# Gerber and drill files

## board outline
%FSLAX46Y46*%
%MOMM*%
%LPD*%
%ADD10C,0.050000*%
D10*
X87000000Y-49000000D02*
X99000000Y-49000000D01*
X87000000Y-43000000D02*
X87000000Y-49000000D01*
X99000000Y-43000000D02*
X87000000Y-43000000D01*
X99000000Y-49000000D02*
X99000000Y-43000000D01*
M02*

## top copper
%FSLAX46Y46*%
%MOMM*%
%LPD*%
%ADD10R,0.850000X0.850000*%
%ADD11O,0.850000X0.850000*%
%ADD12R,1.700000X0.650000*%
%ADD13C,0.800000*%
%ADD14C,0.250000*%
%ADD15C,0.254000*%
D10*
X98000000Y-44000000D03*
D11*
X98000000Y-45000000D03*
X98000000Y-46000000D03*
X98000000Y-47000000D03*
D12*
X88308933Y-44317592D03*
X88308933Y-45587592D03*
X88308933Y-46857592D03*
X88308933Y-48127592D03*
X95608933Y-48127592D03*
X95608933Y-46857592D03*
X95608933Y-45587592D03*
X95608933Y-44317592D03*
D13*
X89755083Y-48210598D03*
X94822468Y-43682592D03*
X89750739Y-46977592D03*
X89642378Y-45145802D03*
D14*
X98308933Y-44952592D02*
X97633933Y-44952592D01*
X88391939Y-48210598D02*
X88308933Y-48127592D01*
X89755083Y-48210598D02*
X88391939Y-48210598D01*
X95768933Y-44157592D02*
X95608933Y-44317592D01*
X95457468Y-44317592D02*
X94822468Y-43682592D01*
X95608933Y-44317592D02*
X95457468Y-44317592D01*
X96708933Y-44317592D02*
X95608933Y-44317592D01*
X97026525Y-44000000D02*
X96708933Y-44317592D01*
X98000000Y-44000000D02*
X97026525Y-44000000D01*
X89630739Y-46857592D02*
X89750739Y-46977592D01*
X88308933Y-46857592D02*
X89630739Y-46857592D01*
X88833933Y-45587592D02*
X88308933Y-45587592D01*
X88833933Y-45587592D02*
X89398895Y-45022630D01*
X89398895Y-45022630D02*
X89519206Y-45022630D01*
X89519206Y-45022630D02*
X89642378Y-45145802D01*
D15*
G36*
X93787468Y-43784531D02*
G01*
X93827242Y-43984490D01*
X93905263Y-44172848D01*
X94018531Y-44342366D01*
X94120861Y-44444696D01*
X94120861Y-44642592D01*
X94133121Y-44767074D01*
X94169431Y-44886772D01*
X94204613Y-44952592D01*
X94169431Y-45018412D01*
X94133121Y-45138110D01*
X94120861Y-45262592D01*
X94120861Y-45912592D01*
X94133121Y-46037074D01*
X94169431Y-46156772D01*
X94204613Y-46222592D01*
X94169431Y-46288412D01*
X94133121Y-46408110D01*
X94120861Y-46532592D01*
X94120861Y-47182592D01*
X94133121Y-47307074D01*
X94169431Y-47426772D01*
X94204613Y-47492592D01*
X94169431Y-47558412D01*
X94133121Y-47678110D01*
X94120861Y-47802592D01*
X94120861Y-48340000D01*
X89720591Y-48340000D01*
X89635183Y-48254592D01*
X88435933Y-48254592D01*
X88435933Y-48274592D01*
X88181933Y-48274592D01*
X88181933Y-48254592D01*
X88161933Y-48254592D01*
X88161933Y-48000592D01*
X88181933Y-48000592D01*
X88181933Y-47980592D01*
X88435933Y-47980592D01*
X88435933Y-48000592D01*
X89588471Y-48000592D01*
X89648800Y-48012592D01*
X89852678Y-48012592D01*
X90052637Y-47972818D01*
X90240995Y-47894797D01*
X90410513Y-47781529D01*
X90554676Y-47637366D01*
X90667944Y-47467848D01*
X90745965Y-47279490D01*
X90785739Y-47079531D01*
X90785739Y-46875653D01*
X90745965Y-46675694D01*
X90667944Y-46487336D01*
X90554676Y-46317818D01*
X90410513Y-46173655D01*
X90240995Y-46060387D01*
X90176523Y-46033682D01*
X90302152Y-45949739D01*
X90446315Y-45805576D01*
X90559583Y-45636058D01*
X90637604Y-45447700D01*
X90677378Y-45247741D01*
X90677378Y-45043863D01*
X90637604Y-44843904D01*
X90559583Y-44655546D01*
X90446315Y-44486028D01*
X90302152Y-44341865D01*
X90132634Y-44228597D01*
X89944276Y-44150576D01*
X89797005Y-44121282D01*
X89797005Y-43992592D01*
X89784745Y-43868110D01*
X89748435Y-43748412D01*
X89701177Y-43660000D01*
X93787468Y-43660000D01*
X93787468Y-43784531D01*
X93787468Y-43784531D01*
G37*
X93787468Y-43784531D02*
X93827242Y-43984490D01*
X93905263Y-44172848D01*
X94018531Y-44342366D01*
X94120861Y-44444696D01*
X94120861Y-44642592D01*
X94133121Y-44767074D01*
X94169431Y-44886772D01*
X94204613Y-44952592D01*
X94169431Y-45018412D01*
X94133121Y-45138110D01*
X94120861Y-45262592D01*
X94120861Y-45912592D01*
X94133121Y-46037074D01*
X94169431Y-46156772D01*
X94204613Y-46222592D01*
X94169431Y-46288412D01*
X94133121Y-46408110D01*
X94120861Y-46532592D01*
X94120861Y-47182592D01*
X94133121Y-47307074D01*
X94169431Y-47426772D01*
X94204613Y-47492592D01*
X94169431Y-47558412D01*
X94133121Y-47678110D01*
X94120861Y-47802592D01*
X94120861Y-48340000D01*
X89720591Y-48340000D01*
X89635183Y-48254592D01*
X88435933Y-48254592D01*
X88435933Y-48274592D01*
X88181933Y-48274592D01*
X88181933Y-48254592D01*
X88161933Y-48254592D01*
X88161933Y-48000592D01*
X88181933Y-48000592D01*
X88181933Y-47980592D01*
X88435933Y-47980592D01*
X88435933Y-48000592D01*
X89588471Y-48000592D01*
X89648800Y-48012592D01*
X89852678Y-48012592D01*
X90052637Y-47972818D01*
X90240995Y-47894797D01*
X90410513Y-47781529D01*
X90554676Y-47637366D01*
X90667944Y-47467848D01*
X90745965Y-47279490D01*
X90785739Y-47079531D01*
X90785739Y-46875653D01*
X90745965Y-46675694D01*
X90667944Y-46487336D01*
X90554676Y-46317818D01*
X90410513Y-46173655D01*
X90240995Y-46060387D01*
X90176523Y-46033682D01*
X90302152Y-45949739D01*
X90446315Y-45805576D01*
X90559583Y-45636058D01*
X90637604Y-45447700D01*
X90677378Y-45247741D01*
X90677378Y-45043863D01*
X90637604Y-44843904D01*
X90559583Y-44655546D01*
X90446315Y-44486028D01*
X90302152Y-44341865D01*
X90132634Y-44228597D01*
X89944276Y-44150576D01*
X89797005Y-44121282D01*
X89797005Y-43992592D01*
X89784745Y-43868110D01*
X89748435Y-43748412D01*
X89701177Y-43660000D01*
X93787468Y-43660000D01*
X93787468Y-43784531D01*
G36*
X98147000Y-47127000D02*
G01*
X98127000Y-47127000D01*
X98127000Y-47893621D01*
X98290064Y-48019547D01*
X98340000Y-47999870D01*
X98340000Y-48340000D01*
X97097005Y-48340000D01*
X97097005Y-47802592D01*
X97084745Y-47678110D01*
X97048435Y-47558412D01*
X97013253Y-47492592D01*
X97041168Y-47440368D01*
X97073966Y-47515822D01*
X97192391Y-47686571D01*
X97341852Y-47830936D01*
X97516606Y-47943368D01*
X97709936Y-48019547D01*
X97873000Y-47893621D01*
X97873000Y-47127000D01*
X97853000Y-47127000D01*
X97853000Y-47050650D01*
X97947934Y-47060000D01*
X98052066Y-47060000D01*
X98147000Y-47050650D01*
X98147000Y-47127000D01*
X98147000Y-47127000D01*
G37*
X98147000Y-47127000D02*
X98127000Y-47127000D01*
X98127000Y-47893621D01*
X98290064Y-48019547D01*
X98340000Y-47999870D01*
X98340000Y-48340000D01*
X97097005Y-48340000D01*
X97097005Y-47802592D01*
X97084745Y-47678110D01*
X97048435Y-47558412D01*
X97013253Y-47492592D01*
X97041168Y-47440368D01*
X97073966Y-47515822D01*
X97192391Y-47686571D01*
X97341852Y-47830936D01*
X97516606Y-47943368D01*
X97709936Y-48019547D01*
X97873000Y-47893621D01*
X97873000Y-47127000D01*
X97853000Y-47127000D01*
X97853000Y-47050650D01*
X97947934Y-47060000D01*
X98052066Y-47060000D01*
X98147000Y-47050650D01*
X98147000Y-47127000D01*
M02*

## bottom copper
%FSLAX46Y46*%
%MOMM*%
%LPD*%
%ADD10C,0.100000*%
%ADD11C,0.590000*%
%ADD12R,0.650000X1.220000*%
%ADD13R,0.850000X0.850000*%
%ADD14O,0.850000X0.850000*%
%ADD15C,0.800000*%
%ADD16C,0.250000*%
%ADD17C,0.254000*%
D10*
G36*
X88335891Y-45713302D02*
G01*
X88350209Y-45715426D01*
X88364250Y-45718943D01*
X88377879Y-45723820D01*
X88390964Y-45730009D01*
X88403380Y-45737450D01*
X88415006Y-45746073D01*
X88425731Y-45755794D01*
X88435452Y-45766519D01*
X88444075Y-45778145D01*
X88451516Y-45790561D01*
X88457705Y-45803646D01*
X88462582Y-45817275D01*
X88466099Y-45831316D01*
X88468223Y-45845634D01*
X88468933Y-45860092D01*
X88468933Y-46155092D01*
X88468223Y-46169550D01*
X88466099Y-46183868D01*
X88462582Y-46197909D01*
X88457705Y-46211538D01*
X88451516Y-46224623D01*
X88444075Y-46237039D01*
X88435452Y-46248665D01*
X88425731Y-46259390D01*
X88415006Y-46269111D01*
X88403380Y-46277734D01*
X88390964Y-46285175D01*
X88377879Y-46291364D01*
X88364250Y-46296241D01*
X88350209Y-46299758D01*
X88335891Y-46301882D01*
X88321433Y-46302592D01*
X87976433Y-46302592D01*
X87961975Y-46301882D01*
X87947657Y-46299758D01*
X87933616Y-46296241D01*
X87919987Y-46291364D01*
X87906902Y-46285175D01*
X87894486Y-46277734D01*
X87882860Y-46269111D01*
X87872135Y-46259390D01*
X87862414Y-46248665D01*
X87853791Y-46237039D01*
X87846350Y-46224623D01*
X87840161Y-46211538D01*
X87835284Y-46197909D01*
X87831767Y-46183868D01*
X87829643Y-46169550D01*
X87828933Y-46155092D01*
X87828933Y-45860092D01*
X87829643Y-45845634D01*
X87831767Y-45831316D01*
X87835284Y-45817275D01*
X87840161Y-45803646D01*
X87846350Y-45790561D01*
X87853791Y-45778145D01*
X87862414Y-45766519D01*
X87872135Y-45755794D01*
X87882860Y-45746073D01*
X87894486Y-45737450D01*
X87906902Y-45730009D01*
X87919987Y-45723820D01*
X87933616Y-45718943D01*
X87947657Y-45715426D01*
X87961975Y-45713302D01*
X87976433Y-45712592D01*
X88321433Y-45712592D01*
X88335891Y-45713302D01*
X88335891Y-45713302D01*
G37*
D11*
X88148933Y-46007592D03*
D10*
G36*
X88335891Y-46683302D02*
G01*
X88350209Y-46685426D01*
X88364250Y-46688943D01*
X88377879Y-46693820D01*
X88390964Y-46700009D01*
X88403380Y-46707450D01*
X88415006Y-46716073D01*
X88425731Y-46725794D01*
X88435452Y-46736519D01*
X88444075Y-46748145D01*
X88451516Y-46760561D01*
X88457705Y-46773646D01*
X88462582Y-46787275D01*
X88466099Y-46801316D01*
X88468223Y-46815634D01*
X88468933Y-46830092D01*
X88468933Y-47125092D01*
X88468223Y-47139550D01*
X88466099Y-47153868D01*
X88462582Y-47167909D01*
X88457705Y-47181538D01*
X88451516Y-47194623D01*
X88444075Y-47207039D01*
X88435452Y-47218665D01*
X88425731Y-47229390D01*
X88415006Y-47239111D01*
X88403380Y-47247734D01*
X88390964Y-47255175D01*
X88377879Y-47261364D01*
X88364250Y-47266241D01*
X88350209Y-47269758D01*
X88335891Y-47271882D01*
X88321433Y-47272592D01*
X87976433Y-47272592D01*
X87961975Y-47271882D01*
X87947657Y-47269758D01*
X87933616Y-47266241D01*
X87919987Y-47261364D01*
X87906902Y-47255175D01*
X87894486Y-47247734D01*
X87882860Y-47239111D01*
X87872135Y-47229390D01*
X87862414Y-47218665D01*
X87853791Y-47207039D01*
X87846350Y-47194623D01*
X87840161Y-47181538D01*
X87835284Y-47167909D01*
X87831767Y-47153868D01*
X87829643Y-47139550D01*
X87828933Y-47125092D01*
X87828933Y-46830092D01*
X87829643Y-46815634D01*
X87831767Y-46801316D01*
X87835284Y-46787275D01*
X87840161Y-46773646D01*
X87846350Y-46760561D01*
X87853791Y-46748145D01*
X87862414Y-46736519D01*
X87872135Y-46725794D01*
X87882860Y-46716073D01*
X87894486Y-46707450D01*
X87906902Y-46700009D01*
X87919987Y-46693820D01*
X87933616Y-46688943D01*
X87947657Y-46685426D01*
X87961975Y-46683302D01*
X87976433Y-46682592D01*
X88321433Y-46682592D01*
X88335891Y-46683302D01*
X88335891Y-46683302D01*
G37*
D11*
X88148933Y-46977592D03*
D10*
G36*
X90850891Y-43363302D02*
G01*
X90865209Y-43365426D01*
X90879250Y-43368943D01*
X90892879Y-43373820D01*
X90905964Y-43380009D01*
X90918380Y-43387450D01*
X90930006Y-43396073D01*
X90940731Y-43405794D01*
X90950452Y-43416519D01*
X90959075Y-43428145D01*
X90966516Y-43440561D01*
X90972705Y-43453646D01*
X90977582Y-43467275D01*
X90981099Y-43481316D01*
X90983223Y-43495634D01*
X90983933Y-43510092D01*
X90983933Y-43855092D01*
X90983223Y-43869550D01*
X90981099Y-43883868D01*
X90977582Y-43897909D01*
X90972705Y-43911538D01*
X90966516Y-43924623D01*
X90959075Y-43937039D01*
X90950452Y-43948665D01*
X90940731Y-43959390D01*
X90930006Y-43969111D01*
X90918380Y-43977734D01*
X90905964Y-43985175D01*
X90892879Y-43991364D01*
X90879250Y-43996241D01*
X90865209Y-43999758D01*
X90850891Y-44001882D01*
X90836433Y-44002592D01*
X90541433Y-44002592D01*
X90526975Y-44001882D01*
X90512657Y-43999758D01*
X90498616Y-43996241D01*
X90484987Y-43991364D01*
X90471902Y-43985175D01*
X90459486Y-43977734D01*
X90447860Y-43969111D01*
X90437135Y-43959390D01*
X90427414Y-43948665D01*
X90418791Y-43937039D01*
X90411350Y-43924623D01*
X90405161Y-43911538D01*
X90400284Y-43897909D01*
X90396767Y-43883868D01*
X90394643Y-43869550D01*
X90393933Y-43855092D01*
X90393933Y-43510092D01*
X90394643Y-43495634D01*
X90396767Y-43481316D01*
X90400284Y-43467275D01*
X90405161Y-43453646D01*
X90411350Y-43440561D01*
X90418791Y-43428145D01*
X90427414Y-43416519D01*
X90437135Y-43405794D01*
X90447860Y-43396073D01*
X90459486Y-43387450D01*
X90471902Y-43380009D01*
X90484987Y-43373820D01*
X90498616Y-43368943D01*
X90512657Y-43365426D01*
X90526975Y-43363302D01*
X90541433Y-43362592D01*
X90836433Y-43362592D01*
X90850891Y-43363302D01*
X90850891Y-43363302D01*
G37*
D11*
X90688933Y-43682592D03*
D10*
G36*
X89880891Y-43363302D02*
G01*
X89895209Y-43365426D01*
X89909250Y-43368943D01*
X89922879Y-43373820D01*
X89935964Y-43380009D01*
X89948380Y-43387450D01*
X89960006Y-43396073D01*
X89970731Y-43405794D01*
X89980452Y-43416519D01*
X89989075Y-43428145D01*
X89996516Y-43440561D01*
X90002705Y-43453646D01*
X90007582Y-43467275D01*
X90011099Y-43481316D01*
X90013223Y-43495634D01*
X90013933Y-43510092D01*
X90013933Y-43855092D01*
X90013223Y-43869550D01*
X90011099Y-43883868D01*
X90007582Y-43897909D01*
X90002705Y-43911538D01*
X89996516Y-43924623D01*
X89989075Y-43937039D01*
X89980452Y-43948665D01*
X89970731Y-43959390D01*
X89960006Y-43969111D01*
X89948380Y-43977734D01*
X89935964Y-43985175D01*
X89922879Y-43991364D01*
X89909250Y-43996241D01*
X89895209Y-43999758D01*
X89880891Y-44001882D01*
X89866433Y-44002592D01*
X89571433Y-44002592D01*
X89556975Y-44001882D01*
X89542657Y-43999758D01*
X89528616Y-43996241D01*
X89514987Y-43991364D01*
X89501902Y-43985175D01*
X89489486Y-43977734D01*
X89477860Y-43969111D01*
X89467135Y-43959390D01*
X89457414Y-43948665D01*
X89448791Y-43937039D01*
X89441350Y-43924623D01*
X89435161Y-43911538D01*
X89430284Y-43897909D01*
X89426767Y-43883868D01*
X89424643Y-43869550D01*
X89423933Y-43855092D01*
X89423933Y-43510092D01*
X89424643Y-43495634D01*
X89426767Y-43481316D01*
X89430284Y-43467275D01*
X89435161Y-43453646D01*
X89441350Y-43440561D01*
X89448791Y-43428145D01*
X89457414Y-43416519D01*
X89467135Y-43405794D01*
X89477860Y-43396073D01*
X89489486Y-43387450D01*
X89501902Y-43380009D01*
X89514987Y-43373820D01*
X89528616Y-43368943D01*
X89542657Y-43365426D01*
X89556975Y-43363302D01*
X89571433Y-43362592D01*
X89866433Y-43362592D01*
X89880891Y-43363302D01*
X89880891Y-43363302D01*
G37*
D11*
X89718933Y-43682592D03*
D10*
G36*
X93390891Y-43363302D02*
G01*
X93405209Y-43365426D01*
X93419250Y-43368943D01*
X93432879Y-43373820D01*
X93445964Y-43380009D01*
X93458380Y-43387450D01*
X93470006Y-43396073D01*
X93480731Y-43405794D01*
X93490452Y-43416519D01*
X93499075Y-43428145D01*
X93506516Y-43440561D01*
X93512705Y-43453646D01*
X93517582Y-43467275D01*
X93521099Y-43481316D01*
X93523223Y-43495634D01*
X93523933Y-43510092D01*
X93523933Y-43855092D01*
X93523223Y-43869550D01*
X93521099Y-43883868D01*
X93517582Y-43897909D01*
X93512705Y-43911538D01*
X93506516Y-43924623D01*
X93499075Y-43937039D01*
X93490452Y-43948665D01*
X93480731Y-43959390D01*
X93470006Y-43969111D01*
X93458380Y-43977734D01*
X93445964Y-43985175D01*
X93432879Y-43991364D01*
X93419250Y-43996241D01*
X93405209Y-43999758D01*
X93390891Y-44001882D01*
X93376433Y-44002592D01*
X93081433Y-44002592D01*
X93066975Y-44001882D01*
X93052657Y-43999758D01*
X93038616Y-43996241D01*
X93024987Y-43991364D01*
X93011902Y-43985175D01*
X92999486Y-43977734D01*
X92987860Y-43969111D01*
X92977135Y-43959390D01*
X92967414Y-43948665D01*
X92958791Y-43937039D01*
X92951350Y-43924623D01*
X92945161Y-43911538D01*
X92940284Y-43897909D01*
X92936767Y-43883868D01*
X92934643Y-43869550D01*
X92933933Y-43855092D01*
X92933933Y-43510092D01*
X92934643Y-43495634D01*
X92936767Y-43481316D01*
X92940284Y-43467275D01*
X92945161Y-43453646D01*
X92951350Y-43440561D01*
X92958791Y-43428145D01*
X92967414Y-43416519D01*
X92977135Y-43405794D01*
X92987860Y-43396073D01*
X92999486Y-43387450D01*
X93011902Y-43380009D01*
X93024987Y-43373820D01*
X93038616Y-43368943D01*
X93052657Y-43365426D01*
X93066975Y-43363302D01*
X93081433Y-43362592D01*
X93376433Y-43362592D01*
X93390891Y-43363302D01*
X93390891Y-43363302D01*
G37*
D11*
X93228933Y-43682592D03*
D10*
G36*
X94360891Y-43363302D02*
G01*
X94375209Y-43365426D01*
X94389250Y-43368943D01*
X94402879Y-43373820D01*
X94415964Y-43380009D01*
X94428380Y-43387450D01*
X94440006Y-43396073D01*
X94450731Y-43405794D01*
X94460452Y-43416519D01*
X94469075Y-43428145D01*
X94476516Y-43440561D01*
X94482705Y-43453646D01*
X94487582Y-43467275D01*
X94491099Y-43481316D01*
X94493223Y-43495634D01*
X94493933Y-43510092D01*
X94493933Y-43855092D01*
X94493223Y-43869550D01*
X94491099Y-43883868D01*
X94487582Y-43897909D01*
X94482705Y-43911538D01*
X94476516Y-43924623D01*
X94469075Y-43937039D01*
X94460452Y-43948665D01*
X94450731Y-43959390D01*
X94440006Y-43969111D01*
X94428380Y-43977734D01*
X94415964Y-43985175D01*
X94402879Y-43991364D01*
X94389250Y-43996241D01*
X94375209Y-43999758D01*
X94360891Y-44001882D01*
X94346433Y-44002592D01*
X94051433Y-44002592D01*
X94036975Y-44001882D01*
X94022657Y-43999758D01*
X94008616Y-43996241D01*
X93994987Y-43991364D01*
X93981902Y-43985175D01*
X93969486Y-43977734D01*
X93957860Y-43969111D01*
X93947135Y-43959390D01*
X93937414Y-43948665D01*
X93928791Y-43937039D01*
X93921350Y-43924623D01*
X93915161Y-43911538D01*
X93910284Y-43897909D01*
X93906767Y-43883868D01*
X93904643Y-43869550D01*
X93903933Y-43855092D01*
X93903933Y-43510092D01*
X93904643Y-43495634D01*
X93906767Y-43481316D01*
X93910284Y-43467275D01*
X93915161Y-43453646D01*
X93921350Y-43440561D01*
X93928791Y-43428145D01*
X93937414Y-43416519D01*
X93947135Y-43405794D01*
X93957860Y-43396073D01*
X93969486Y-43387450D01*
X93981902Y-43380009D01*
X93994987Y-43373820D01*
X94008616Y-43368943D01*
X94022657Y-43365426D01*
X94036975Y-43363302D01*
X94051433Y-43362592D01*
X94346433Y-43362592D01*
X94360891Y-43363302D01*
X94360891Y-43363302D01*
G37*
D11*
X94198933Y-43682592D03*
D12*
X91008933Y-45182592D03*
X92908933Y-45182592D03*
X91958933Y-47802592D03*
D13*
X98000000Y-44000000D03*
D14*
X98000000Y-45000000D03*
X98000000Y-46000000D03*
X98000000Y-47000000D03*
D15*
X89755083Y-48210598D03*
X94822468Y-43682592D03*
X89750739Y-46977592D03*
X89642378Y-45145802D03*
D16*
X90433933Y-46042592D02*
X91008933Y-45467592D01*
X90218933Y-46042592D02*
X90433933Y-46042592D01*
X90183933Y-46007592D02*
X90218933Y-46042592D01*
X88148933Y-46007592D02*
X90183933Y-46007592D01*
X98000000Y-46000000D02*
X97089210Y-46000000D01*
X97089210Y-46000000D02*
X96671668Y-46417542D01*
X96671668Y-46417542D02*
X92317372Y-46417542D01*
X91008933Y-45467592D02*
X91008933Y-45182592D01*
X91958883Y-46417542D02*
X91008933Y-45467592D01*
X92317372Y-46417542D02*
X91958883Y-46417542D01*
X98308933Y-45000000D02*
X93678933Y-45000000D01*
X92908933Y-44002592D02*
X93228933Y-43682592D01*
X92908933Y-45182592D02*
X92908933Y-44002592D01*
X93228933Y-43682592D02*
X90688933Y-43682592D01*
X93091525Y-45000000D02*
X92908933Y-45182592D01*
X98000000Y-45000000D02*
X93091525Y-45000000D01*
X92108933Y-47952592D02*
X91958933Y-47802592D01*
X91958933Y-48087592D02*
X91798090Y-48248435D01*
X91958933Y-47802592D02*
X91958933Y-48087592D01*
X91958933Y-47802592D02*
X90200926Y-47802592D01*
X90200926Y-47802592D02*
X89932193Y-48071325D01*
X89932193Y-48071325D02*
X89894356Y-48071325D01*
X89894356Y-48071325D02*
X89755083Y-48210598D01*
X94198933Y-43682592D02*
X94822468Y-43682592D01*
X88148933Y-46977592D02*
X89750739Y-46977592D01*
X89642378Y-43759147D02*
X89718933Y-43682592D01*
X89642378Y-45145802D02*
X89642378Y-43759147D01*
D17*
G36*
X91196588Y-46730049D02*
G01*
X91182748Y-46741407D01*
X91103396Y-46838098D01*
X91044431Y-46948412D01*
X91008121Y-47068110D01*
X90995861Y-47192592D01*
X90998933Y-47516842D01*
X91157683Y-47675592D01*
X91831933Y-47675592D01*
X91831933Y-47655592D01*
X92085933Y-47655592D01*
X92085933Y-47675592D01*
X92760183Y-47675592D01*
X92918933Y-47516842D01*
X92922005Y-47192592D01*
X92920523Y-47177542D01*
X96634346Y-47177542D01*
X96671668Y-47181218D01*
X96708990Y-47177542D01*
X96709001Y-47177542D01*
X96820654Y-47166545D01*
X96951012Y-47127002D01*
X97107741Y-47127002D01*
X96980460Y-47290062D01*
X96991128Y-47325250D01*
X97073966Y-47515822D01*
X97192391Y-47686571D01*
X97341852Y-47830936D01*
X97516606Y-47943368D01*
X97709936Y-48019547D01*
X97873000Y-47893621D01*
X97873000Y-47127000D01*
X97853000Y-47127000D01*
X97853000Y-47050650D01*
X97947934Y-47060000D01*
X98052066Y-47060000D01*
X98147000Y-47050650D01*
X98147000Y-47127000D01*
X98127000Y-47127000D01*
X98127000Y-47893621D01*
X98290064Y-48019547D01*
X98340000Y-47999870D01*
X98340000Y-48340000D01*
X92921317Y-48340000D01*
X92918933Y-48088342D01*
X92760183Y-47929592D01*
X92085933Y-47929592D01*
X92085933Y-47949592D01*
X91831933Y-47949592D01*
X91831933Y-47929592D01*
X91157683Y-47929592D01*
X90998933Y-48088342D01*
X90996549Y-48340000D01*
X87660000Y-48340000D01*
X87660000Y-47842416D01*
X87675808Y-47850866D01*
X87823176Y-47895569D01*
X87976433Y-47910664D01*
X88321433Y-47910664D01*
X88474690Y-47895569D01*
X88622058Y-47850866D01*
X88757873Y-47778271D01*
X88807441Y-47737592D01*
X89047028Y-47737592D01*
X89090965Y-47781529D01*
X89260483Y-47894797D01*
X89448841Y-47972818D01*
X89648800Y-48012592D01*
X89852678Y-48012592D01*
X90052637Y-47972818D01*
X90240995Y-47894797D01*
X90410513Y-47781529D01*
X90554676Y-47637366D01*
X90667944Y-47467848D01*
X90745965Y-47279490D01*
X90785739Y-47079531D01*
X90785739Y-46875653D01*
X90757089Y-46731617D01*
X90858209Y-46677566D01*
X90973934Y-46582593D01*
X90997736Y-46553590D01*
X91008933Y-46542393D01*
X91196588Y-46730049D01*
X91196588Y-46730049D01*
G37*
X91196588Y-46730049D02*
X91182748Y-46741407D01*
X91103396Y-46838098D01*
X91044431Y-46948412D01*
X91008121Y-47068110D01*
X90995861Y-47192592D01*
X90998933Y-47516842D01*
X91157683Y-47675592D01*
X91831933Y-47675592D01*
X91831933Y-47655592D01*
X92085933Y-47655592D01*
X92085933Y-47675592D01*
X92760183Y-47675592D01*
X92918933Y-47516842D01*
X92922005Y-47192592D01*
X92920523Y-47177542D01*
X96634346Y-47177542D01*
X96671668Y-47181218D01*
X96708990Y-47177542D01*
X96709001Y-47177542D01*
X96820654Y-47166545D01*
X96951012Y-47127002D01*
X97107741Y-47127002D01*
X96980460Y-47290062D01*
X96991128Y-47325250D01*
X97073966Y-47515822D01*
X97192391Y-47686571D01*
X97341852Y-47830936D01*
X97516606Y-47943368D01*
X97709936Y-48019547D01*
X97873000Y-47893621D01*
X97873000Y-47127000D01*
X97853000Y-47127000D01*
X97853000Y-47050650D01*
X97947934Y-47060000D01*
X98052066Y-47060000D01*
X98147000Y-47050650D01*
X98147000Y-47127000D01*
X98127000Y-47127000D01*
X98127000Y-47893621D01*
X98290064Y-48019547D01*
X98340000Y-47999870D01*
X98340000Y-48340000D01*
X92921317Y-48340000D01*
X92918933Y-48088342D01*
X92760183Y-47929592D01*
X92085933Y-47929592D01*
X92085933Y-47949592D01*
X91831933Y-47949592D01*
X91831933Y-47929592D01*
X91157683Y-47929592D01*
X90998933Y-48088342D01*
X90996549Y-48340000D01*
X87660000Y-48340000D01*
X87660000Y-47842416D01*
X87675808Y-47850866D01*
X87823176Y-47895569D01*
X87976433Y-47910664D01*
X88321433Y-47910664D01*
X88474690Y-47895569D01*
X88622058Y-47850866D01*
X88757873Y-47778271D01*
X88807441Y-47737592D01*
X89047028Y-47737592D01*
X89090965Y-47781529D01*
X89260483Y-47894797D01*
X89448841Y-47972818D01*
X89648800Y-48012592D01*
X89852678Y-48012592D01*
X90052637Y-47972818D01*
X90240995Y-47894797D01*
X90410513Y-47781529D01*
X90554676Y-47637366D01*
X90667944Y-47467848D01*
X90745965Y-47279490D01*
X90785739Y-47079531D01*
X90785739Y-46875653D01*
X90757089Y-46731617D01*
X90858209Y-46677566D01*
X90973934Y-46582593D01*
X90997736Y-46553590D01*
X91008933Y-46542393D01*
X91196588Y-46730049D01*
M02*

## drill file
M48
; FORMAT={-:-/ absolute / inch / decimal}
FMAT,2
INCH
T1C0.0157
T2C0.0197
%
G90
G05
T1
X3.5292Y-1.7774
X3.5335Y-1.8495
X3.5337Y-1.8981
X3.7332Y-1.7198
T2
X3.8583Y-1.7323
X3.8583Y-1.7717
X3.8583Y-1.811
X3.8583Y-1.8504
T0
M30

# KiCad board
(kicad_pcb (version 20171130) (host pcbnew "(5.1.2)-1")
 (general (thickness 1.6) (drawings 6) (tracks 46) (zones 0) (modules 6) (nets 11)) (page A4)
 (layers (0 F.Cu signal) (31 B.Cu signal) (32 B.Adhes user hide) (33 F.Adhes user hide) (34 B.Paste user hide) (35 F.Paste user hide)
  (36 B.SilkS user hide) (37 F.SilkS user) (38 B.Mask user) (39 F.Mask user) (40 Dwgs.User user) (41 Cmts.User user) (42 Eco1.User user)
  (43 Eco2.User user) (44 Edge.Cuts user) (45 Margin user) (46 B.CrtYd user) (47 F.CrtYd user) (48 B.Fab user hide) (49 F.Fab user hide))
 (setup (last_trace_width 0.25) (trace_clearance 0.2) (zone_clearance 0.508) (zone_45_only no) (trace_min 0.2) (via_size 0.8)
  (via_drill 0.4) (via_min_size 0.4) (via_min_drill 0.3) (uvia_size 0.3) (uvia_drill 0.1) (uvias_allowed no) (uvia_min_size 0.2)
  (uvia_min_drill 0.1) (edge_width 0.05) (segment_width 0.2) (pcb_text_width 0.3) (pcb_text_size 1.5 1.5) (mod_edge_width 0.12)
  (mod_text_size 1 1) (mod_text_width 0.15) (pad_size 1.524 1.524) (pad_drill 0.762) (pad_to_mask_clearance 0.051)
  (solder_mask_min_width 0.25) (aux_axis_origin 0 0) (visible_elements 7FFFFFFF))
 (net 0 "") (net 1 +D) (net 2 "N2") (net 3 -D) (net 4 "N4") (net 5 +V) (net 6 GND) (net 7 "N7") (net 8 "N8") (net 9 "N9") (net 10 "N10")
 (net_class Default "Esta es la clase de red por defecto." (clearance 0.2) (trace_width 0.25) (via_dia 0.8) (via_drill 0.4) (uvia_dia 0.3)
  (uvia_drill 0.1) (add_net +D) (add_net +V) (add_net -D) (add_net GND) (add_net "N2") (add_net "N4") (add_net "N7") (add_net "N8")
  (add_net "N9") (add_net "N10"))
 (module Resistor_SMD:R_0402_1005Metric (layer B.Cu) (at 88.148933 46.492592 90)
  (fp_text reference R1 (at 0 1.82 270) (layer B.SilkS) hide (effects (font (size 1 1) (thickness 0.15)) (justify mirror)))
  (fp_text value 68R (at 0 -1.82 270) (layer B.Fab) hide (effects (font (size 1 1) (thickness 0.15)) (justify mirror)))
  (pad 2 smd roundrect (at 0.485 0 90) (size 0.59 0.64) (layers B.Cu B.Paste B.Mask) (roundrect_rratio 0.25) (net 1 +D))
  (pad 1 smd roundrect (at -0.485 0 90) (size 0.59 0.64) (layers B.Cu B.Paste B.Mask) (roundrect_rratio 0.25) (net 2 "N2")))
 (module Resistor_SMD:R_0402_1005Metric (layer B.Cu) (at 90.203933 43.682592)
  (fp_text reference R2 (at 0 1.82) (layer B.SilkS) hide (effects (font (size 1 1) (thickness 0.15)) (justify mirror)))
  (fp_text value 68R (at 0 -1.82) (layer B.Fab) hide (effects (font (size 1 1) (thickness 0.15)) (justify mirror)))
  (pad 2 smd roundrect (at 0.485 0) (size 0.59 0.64) (layers B.Cu B.Paste B.Mask) (roundrect_rratio 0.25) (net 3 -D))
  (pad 1 smd roundrect (at -0.485 0) (size 0.59 0.64) (layers B.Cu B.Paste B.Mask) (roundrect_rratio 0.25) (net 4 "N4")))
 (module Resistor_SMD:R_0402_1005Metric (layer B.Cu) (at 93.713933 43.682592 180)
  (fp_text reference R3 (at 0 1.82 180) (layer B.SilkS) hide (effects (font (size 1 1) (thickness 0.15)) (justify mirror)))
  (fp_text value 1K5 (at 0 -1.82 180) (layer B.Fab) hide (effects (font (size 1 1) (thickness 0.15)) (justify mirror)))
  (pad 2 smd roundrect (at 0.485 0 180) (size 0.59 0.64) (layers B.Cu B.Paste B.Mask) (roundrect_rratio 0.25) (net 3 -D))
  (pad 1 smd roundrect (at -0.485 0 180) (size 0.59 0.64) (layers B.Cu B.Paste B.Mask) (roundrect_rratio 0.25) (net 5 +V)))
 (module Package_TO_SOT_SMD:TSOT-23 (layer B.Cu) (at 91.958933 46.492592 270)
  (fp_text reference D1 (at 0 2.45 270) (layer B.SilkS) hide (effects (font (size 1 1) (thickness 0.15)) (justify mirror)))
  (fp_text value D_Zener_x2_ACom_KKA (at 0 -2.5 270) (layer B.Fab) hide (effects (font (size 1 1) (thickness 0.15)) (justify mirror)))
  (pad 1 smd rect (at -1.31 0.95 270) (size 1.22 0.65) (layers B.Cu B.Paste B.Mask) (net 1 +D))
  (pad 2 smd rect (at -1.31 -0.95 270) (size 1.22 0.65) (layers B.Cu B.Paste B.Mask) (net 3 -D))
  (pad 3 smd rect (at 1.31 0 270) (size 1.22 0.65) (layers B.Cu B.Paste B.Mask) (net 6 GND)))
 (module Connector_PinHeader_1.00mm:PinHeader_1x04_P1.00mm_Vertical (layer F.Cu) (at 98 44)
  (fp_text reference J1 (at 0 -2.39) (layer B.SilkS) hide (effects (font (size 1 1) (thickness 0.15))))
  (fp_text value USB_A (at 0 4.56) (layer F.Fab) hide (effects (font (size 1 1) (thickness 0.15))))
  (pad 1 thru_hole rect (at 0 0) (size 0.85 0.85) (drill 0.5) (layers *.Cu *.Mask) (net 5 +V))
  (pad 2 thru_hole oval (at 0 1) (size 0.85 0.85) (drill 0.5) (layers *.Cu *.Mask) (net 3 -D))
  (pad 3 thru_hole oval (at 0 2) (size 0.85 0.85) (drill 0.5) (layers *.Cu *.Mask) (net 1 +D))
  (pad 4 thru_hole oval (at 0 3) (size 0.85 0.85) (drill 0.5) (layers *.Cu *.Mask) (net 6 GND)))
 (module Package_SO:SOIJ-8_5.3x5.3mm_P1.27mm (layer F.Cu) (at 91.958933 46.222592)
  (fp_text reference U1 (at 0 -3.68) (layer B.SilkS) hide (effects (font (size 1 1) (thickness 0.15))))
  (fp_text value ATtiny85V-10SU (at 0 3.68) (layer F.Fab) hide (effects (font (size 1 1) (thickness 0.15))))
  (pad 1 smd rect (at -3.65 -1.905) (size 1.7 0.65) (layers F.Cu F.Paste F.Mask) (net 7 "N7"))
  (pad 2 smd rect (at -3.65 -0.635) (size 1.7 0.65) (layers F.Cu F.Paste F.Mask) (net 4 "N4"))
  (pad 3 smd rect (at -3.65 0.635) (size 1.7 0.65) (layers F.Cu F.Paste F.Mask) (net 2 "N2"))
  (pad 4 smd rect (at -3.65 1.905) (size 1.7 0.65) (layers F.Cu F.Paste F.Mask) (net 6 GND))
  (pad 5 smd rect (at 3.65 1.905) (size 1.7 0.65) (layers F.Cu F.Paste F.Mask) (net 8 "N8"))
  (pad 6 smd rect (at 3.65 0.635) (size 1.7 0.65) (layers F.Cu F.Paste F.Mask) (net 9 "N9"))
  (pad 7 smd rect (at 3.65 -0.635) (size 1.7 0.65) (layers F.Cu F.Paste F.Mask) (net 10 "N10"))
  (pad 8 smd rect (at 3.65 -1.905) (size 1.7 0.65) (layers F.Cu F.Paste F.Mask) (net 5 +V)))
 (gr_line (start 87 49) (end 99 49) (layer Edge.Cuts) (width 0.05))
 (gr_line (start 87 43) (end 87 49) (layer Edge.Cuts) (width 0.05))
 (gr_line (start 99 43) (end 87 43) (layer Edge.Cuts) (width 0.05))
 (gr_line (start 99 49) (end 99 43) (layer Edge.Cuts) (width 0.05))
 (segment (start 90.433933 46.042592) (end 91.008933 45.467592) (width 0.25) (layer B.Cu) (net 1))
 (segment (start 90.218933 46.042592) (end 90.433933 46.042592) (width 0.25) (layer B.Cu) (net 1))
 (segment (start 90.183933 46.007592) (end 90.218933 46.042592) (width 0.25) (layer B.Cu) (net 1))
 (segment (start 88.148933 46.007592) (end 90.183933 46.007592) (width 0.25) (layer B.Cu) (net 1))
 (segment (start 98 46) (end 97.08921 46) (width 0.25) (layer B.Cu) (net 1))
 (segment (start 97.08921 46) (end 96.671668 46.417542) (width 0.25) (layer B.Cu) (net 1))
 (segment (start 96.671668 46.417542) (end 92.317372 46.417542) (width 0.25) (layer B.Cu) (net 1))
 (segment (start 91.008933 45.467592) (end 91.008933 45.182592) (width 0.25) (layer B.Cu) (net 1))
 (segment (start 91.958883 46.417542) (end 91.008933 45.467592) (width 0.25) (layer B.Cu) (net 1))
 (segment (start 92.317372 46.417542) (end 91.958883 46.417542) (width 0.25) (layer B.Cu) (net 1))
 (segment (start 98.308933 45) (end 93.678933 45) (width 0.25) (layer B.Cu) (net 3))
 (segment (start 92.908933 44.002592) (end 93.228933 43.682592) (width 0.25) (layer B.Cu) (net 3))
 (segment (start 92.908933 45.182592) (end 92.908933 44.002592) (width 0.25) (layer B.Cu) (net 3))
 (segment (start 93.228933 43.682592) (end 90.688933 43.682592) (width 0.25) (layer B.Cu) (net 3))
 (segment (start 93.091525 45) (end 92.908933 45.182592) (width 0.25) (layer B.Cu) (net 3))
 (segment (start 98 45) (end 93.091525 45) (width 0.25) (layer B.Cu) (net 3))
 (segment (start 98.308933 44.952592) (end 97.633933 44.952592) (width 0.25) (layer F.Cu) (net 3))
 (segment (start 92.108933 47.952592) (end 91.958933 47.802592) (width 0.25) (layer B.Cu) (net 6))
 (segment (start 91.958933 48.087592) (end 91.79809 48.248435) (width 0.25) (layer B.Cu) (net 6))
 (segment (start 91.958933 47.802592) (end 91.958933 48.087592) (width 0.25) (layer B.Cu) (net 6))
 (segment (start 91.958933 47.802592) (end 90.200926 47.802592) (width 0.25) (layer B.Cu) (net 6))
 (segment (start 90.200926 47.802592) (end 89.932193 48.071325) (width 0.25) (layer B.Cu) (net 6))
 (via (at 89.755083 48.210598) (size 0.8) (drill 0.4) (layers F.Cu B.Cu) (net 6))
 (segment (start 89.932193 48.071325) (end 89.894356 48.071325) (width 0.25) (layer B.Cu) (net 6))
 (segment (start 89.894356 48.071325) (end 89.755083 48.210598) (width 0.25) (layer B.Cu) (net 6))
 (segment (start 88.391939 48.210598) (end 88.308933 48.127592) (width 0.25) (layer F.Cu) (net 6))
 (segment (start 89.755083 48.210598) (end 88.391939 48.210598) (width 0.25) (layer F.Cu) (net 6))
 (segment (start 95.768933 44.157592) (end 95.608933 44.317592) (width 0.25) (layer F.Cu) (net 5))
 (segment (start 94.198933 43.682592) (end 94.822468 43.682592) (width 0.25) (layer B.Cu) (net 5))
 (via (at 94.822468 43.682592) (size 0.8) (drill 0.4) (layers F.Cu B.Cu) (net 5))
 (segment (start 95.457468 44.317592) (end 94.822468 43.682592) (width 0.25) (layer F.Cu) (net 5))
 (segment (start 95.608933 44.317592) (end 95.457468 44.317592) (width 0.25) (layer F.Cu) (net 5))
 (segment (start 96.708933 44.317592) (end 95.608933 44.317592) (width 0.25) (layer F.Cu) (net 5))
 (segment (start 97.026525 44) (end 96.708933 44.317592) (width 0.25) (layer F.Cu) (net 5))
 (segment (start 98 44) (end 97.026525 44) (width 0.25) (layer F.Cu) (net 5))
 (segment (start 88.148933 46.977592) (end 89.750739 46.977592) (width 0.25) (layer B.Cu) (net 2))
 (via (at 89.750739 46.977592) (size 0.8) (drill 0.4) (layers F.Cu B.Cu) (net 2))
 (segment (start 89.630739 46.857592) (end 89.750739 46.977592) (width 0.25) (layer F.Cu) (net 2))
 (segment (start 88.308933 46.857592) (end 89.630739 46.857592) (width 0.25) (layer F.Cu) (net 2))
 (segment (start 88.833933 45.587592) (end 88.308933 45.587592) (width 0.25) (layer F.Cu) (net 4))
 (segment (start 88.833933 45.587592) (end 89.398895 45.02263) (width 0.25) (layer F.Cu) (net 4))
 (via (at 89.642378 45.145802) (size 0.8) (drill 0.4) (layers F.Cu B.Cu) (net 4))
 (segment (start 89.398895 45.02263) (end 89.519206 45.02263) (width 0.25) (layer F.Cu) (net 4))
 (segment (start 89.519206 45.02263) (end 89.642378 45.145802) (width 0.25) (layer F.Cu) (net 4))
 (segment (start 89.642378 43.759147) (end 89.718933 43.682592) (width 0.25) (layer B.Cu) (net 4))
 (segment (start 89.642378 45.145802) (end 89.642378 43.759147) (width 0.25) (layer B.Cu) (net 4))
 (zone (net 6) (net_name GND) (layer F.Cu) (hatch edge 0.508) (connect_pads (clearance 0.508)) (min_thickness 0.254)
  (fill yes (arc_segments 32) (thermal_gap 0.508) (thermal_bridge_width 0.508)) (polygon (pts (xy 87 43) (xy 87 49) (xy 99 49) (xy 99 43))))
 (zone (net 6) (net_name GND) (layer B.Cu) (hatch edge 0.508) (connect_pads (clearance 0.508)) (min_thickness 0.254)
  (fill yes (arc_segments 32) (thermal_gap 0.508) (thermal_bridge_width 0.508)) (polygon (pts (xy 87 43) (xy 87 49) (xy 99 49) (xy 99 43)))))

